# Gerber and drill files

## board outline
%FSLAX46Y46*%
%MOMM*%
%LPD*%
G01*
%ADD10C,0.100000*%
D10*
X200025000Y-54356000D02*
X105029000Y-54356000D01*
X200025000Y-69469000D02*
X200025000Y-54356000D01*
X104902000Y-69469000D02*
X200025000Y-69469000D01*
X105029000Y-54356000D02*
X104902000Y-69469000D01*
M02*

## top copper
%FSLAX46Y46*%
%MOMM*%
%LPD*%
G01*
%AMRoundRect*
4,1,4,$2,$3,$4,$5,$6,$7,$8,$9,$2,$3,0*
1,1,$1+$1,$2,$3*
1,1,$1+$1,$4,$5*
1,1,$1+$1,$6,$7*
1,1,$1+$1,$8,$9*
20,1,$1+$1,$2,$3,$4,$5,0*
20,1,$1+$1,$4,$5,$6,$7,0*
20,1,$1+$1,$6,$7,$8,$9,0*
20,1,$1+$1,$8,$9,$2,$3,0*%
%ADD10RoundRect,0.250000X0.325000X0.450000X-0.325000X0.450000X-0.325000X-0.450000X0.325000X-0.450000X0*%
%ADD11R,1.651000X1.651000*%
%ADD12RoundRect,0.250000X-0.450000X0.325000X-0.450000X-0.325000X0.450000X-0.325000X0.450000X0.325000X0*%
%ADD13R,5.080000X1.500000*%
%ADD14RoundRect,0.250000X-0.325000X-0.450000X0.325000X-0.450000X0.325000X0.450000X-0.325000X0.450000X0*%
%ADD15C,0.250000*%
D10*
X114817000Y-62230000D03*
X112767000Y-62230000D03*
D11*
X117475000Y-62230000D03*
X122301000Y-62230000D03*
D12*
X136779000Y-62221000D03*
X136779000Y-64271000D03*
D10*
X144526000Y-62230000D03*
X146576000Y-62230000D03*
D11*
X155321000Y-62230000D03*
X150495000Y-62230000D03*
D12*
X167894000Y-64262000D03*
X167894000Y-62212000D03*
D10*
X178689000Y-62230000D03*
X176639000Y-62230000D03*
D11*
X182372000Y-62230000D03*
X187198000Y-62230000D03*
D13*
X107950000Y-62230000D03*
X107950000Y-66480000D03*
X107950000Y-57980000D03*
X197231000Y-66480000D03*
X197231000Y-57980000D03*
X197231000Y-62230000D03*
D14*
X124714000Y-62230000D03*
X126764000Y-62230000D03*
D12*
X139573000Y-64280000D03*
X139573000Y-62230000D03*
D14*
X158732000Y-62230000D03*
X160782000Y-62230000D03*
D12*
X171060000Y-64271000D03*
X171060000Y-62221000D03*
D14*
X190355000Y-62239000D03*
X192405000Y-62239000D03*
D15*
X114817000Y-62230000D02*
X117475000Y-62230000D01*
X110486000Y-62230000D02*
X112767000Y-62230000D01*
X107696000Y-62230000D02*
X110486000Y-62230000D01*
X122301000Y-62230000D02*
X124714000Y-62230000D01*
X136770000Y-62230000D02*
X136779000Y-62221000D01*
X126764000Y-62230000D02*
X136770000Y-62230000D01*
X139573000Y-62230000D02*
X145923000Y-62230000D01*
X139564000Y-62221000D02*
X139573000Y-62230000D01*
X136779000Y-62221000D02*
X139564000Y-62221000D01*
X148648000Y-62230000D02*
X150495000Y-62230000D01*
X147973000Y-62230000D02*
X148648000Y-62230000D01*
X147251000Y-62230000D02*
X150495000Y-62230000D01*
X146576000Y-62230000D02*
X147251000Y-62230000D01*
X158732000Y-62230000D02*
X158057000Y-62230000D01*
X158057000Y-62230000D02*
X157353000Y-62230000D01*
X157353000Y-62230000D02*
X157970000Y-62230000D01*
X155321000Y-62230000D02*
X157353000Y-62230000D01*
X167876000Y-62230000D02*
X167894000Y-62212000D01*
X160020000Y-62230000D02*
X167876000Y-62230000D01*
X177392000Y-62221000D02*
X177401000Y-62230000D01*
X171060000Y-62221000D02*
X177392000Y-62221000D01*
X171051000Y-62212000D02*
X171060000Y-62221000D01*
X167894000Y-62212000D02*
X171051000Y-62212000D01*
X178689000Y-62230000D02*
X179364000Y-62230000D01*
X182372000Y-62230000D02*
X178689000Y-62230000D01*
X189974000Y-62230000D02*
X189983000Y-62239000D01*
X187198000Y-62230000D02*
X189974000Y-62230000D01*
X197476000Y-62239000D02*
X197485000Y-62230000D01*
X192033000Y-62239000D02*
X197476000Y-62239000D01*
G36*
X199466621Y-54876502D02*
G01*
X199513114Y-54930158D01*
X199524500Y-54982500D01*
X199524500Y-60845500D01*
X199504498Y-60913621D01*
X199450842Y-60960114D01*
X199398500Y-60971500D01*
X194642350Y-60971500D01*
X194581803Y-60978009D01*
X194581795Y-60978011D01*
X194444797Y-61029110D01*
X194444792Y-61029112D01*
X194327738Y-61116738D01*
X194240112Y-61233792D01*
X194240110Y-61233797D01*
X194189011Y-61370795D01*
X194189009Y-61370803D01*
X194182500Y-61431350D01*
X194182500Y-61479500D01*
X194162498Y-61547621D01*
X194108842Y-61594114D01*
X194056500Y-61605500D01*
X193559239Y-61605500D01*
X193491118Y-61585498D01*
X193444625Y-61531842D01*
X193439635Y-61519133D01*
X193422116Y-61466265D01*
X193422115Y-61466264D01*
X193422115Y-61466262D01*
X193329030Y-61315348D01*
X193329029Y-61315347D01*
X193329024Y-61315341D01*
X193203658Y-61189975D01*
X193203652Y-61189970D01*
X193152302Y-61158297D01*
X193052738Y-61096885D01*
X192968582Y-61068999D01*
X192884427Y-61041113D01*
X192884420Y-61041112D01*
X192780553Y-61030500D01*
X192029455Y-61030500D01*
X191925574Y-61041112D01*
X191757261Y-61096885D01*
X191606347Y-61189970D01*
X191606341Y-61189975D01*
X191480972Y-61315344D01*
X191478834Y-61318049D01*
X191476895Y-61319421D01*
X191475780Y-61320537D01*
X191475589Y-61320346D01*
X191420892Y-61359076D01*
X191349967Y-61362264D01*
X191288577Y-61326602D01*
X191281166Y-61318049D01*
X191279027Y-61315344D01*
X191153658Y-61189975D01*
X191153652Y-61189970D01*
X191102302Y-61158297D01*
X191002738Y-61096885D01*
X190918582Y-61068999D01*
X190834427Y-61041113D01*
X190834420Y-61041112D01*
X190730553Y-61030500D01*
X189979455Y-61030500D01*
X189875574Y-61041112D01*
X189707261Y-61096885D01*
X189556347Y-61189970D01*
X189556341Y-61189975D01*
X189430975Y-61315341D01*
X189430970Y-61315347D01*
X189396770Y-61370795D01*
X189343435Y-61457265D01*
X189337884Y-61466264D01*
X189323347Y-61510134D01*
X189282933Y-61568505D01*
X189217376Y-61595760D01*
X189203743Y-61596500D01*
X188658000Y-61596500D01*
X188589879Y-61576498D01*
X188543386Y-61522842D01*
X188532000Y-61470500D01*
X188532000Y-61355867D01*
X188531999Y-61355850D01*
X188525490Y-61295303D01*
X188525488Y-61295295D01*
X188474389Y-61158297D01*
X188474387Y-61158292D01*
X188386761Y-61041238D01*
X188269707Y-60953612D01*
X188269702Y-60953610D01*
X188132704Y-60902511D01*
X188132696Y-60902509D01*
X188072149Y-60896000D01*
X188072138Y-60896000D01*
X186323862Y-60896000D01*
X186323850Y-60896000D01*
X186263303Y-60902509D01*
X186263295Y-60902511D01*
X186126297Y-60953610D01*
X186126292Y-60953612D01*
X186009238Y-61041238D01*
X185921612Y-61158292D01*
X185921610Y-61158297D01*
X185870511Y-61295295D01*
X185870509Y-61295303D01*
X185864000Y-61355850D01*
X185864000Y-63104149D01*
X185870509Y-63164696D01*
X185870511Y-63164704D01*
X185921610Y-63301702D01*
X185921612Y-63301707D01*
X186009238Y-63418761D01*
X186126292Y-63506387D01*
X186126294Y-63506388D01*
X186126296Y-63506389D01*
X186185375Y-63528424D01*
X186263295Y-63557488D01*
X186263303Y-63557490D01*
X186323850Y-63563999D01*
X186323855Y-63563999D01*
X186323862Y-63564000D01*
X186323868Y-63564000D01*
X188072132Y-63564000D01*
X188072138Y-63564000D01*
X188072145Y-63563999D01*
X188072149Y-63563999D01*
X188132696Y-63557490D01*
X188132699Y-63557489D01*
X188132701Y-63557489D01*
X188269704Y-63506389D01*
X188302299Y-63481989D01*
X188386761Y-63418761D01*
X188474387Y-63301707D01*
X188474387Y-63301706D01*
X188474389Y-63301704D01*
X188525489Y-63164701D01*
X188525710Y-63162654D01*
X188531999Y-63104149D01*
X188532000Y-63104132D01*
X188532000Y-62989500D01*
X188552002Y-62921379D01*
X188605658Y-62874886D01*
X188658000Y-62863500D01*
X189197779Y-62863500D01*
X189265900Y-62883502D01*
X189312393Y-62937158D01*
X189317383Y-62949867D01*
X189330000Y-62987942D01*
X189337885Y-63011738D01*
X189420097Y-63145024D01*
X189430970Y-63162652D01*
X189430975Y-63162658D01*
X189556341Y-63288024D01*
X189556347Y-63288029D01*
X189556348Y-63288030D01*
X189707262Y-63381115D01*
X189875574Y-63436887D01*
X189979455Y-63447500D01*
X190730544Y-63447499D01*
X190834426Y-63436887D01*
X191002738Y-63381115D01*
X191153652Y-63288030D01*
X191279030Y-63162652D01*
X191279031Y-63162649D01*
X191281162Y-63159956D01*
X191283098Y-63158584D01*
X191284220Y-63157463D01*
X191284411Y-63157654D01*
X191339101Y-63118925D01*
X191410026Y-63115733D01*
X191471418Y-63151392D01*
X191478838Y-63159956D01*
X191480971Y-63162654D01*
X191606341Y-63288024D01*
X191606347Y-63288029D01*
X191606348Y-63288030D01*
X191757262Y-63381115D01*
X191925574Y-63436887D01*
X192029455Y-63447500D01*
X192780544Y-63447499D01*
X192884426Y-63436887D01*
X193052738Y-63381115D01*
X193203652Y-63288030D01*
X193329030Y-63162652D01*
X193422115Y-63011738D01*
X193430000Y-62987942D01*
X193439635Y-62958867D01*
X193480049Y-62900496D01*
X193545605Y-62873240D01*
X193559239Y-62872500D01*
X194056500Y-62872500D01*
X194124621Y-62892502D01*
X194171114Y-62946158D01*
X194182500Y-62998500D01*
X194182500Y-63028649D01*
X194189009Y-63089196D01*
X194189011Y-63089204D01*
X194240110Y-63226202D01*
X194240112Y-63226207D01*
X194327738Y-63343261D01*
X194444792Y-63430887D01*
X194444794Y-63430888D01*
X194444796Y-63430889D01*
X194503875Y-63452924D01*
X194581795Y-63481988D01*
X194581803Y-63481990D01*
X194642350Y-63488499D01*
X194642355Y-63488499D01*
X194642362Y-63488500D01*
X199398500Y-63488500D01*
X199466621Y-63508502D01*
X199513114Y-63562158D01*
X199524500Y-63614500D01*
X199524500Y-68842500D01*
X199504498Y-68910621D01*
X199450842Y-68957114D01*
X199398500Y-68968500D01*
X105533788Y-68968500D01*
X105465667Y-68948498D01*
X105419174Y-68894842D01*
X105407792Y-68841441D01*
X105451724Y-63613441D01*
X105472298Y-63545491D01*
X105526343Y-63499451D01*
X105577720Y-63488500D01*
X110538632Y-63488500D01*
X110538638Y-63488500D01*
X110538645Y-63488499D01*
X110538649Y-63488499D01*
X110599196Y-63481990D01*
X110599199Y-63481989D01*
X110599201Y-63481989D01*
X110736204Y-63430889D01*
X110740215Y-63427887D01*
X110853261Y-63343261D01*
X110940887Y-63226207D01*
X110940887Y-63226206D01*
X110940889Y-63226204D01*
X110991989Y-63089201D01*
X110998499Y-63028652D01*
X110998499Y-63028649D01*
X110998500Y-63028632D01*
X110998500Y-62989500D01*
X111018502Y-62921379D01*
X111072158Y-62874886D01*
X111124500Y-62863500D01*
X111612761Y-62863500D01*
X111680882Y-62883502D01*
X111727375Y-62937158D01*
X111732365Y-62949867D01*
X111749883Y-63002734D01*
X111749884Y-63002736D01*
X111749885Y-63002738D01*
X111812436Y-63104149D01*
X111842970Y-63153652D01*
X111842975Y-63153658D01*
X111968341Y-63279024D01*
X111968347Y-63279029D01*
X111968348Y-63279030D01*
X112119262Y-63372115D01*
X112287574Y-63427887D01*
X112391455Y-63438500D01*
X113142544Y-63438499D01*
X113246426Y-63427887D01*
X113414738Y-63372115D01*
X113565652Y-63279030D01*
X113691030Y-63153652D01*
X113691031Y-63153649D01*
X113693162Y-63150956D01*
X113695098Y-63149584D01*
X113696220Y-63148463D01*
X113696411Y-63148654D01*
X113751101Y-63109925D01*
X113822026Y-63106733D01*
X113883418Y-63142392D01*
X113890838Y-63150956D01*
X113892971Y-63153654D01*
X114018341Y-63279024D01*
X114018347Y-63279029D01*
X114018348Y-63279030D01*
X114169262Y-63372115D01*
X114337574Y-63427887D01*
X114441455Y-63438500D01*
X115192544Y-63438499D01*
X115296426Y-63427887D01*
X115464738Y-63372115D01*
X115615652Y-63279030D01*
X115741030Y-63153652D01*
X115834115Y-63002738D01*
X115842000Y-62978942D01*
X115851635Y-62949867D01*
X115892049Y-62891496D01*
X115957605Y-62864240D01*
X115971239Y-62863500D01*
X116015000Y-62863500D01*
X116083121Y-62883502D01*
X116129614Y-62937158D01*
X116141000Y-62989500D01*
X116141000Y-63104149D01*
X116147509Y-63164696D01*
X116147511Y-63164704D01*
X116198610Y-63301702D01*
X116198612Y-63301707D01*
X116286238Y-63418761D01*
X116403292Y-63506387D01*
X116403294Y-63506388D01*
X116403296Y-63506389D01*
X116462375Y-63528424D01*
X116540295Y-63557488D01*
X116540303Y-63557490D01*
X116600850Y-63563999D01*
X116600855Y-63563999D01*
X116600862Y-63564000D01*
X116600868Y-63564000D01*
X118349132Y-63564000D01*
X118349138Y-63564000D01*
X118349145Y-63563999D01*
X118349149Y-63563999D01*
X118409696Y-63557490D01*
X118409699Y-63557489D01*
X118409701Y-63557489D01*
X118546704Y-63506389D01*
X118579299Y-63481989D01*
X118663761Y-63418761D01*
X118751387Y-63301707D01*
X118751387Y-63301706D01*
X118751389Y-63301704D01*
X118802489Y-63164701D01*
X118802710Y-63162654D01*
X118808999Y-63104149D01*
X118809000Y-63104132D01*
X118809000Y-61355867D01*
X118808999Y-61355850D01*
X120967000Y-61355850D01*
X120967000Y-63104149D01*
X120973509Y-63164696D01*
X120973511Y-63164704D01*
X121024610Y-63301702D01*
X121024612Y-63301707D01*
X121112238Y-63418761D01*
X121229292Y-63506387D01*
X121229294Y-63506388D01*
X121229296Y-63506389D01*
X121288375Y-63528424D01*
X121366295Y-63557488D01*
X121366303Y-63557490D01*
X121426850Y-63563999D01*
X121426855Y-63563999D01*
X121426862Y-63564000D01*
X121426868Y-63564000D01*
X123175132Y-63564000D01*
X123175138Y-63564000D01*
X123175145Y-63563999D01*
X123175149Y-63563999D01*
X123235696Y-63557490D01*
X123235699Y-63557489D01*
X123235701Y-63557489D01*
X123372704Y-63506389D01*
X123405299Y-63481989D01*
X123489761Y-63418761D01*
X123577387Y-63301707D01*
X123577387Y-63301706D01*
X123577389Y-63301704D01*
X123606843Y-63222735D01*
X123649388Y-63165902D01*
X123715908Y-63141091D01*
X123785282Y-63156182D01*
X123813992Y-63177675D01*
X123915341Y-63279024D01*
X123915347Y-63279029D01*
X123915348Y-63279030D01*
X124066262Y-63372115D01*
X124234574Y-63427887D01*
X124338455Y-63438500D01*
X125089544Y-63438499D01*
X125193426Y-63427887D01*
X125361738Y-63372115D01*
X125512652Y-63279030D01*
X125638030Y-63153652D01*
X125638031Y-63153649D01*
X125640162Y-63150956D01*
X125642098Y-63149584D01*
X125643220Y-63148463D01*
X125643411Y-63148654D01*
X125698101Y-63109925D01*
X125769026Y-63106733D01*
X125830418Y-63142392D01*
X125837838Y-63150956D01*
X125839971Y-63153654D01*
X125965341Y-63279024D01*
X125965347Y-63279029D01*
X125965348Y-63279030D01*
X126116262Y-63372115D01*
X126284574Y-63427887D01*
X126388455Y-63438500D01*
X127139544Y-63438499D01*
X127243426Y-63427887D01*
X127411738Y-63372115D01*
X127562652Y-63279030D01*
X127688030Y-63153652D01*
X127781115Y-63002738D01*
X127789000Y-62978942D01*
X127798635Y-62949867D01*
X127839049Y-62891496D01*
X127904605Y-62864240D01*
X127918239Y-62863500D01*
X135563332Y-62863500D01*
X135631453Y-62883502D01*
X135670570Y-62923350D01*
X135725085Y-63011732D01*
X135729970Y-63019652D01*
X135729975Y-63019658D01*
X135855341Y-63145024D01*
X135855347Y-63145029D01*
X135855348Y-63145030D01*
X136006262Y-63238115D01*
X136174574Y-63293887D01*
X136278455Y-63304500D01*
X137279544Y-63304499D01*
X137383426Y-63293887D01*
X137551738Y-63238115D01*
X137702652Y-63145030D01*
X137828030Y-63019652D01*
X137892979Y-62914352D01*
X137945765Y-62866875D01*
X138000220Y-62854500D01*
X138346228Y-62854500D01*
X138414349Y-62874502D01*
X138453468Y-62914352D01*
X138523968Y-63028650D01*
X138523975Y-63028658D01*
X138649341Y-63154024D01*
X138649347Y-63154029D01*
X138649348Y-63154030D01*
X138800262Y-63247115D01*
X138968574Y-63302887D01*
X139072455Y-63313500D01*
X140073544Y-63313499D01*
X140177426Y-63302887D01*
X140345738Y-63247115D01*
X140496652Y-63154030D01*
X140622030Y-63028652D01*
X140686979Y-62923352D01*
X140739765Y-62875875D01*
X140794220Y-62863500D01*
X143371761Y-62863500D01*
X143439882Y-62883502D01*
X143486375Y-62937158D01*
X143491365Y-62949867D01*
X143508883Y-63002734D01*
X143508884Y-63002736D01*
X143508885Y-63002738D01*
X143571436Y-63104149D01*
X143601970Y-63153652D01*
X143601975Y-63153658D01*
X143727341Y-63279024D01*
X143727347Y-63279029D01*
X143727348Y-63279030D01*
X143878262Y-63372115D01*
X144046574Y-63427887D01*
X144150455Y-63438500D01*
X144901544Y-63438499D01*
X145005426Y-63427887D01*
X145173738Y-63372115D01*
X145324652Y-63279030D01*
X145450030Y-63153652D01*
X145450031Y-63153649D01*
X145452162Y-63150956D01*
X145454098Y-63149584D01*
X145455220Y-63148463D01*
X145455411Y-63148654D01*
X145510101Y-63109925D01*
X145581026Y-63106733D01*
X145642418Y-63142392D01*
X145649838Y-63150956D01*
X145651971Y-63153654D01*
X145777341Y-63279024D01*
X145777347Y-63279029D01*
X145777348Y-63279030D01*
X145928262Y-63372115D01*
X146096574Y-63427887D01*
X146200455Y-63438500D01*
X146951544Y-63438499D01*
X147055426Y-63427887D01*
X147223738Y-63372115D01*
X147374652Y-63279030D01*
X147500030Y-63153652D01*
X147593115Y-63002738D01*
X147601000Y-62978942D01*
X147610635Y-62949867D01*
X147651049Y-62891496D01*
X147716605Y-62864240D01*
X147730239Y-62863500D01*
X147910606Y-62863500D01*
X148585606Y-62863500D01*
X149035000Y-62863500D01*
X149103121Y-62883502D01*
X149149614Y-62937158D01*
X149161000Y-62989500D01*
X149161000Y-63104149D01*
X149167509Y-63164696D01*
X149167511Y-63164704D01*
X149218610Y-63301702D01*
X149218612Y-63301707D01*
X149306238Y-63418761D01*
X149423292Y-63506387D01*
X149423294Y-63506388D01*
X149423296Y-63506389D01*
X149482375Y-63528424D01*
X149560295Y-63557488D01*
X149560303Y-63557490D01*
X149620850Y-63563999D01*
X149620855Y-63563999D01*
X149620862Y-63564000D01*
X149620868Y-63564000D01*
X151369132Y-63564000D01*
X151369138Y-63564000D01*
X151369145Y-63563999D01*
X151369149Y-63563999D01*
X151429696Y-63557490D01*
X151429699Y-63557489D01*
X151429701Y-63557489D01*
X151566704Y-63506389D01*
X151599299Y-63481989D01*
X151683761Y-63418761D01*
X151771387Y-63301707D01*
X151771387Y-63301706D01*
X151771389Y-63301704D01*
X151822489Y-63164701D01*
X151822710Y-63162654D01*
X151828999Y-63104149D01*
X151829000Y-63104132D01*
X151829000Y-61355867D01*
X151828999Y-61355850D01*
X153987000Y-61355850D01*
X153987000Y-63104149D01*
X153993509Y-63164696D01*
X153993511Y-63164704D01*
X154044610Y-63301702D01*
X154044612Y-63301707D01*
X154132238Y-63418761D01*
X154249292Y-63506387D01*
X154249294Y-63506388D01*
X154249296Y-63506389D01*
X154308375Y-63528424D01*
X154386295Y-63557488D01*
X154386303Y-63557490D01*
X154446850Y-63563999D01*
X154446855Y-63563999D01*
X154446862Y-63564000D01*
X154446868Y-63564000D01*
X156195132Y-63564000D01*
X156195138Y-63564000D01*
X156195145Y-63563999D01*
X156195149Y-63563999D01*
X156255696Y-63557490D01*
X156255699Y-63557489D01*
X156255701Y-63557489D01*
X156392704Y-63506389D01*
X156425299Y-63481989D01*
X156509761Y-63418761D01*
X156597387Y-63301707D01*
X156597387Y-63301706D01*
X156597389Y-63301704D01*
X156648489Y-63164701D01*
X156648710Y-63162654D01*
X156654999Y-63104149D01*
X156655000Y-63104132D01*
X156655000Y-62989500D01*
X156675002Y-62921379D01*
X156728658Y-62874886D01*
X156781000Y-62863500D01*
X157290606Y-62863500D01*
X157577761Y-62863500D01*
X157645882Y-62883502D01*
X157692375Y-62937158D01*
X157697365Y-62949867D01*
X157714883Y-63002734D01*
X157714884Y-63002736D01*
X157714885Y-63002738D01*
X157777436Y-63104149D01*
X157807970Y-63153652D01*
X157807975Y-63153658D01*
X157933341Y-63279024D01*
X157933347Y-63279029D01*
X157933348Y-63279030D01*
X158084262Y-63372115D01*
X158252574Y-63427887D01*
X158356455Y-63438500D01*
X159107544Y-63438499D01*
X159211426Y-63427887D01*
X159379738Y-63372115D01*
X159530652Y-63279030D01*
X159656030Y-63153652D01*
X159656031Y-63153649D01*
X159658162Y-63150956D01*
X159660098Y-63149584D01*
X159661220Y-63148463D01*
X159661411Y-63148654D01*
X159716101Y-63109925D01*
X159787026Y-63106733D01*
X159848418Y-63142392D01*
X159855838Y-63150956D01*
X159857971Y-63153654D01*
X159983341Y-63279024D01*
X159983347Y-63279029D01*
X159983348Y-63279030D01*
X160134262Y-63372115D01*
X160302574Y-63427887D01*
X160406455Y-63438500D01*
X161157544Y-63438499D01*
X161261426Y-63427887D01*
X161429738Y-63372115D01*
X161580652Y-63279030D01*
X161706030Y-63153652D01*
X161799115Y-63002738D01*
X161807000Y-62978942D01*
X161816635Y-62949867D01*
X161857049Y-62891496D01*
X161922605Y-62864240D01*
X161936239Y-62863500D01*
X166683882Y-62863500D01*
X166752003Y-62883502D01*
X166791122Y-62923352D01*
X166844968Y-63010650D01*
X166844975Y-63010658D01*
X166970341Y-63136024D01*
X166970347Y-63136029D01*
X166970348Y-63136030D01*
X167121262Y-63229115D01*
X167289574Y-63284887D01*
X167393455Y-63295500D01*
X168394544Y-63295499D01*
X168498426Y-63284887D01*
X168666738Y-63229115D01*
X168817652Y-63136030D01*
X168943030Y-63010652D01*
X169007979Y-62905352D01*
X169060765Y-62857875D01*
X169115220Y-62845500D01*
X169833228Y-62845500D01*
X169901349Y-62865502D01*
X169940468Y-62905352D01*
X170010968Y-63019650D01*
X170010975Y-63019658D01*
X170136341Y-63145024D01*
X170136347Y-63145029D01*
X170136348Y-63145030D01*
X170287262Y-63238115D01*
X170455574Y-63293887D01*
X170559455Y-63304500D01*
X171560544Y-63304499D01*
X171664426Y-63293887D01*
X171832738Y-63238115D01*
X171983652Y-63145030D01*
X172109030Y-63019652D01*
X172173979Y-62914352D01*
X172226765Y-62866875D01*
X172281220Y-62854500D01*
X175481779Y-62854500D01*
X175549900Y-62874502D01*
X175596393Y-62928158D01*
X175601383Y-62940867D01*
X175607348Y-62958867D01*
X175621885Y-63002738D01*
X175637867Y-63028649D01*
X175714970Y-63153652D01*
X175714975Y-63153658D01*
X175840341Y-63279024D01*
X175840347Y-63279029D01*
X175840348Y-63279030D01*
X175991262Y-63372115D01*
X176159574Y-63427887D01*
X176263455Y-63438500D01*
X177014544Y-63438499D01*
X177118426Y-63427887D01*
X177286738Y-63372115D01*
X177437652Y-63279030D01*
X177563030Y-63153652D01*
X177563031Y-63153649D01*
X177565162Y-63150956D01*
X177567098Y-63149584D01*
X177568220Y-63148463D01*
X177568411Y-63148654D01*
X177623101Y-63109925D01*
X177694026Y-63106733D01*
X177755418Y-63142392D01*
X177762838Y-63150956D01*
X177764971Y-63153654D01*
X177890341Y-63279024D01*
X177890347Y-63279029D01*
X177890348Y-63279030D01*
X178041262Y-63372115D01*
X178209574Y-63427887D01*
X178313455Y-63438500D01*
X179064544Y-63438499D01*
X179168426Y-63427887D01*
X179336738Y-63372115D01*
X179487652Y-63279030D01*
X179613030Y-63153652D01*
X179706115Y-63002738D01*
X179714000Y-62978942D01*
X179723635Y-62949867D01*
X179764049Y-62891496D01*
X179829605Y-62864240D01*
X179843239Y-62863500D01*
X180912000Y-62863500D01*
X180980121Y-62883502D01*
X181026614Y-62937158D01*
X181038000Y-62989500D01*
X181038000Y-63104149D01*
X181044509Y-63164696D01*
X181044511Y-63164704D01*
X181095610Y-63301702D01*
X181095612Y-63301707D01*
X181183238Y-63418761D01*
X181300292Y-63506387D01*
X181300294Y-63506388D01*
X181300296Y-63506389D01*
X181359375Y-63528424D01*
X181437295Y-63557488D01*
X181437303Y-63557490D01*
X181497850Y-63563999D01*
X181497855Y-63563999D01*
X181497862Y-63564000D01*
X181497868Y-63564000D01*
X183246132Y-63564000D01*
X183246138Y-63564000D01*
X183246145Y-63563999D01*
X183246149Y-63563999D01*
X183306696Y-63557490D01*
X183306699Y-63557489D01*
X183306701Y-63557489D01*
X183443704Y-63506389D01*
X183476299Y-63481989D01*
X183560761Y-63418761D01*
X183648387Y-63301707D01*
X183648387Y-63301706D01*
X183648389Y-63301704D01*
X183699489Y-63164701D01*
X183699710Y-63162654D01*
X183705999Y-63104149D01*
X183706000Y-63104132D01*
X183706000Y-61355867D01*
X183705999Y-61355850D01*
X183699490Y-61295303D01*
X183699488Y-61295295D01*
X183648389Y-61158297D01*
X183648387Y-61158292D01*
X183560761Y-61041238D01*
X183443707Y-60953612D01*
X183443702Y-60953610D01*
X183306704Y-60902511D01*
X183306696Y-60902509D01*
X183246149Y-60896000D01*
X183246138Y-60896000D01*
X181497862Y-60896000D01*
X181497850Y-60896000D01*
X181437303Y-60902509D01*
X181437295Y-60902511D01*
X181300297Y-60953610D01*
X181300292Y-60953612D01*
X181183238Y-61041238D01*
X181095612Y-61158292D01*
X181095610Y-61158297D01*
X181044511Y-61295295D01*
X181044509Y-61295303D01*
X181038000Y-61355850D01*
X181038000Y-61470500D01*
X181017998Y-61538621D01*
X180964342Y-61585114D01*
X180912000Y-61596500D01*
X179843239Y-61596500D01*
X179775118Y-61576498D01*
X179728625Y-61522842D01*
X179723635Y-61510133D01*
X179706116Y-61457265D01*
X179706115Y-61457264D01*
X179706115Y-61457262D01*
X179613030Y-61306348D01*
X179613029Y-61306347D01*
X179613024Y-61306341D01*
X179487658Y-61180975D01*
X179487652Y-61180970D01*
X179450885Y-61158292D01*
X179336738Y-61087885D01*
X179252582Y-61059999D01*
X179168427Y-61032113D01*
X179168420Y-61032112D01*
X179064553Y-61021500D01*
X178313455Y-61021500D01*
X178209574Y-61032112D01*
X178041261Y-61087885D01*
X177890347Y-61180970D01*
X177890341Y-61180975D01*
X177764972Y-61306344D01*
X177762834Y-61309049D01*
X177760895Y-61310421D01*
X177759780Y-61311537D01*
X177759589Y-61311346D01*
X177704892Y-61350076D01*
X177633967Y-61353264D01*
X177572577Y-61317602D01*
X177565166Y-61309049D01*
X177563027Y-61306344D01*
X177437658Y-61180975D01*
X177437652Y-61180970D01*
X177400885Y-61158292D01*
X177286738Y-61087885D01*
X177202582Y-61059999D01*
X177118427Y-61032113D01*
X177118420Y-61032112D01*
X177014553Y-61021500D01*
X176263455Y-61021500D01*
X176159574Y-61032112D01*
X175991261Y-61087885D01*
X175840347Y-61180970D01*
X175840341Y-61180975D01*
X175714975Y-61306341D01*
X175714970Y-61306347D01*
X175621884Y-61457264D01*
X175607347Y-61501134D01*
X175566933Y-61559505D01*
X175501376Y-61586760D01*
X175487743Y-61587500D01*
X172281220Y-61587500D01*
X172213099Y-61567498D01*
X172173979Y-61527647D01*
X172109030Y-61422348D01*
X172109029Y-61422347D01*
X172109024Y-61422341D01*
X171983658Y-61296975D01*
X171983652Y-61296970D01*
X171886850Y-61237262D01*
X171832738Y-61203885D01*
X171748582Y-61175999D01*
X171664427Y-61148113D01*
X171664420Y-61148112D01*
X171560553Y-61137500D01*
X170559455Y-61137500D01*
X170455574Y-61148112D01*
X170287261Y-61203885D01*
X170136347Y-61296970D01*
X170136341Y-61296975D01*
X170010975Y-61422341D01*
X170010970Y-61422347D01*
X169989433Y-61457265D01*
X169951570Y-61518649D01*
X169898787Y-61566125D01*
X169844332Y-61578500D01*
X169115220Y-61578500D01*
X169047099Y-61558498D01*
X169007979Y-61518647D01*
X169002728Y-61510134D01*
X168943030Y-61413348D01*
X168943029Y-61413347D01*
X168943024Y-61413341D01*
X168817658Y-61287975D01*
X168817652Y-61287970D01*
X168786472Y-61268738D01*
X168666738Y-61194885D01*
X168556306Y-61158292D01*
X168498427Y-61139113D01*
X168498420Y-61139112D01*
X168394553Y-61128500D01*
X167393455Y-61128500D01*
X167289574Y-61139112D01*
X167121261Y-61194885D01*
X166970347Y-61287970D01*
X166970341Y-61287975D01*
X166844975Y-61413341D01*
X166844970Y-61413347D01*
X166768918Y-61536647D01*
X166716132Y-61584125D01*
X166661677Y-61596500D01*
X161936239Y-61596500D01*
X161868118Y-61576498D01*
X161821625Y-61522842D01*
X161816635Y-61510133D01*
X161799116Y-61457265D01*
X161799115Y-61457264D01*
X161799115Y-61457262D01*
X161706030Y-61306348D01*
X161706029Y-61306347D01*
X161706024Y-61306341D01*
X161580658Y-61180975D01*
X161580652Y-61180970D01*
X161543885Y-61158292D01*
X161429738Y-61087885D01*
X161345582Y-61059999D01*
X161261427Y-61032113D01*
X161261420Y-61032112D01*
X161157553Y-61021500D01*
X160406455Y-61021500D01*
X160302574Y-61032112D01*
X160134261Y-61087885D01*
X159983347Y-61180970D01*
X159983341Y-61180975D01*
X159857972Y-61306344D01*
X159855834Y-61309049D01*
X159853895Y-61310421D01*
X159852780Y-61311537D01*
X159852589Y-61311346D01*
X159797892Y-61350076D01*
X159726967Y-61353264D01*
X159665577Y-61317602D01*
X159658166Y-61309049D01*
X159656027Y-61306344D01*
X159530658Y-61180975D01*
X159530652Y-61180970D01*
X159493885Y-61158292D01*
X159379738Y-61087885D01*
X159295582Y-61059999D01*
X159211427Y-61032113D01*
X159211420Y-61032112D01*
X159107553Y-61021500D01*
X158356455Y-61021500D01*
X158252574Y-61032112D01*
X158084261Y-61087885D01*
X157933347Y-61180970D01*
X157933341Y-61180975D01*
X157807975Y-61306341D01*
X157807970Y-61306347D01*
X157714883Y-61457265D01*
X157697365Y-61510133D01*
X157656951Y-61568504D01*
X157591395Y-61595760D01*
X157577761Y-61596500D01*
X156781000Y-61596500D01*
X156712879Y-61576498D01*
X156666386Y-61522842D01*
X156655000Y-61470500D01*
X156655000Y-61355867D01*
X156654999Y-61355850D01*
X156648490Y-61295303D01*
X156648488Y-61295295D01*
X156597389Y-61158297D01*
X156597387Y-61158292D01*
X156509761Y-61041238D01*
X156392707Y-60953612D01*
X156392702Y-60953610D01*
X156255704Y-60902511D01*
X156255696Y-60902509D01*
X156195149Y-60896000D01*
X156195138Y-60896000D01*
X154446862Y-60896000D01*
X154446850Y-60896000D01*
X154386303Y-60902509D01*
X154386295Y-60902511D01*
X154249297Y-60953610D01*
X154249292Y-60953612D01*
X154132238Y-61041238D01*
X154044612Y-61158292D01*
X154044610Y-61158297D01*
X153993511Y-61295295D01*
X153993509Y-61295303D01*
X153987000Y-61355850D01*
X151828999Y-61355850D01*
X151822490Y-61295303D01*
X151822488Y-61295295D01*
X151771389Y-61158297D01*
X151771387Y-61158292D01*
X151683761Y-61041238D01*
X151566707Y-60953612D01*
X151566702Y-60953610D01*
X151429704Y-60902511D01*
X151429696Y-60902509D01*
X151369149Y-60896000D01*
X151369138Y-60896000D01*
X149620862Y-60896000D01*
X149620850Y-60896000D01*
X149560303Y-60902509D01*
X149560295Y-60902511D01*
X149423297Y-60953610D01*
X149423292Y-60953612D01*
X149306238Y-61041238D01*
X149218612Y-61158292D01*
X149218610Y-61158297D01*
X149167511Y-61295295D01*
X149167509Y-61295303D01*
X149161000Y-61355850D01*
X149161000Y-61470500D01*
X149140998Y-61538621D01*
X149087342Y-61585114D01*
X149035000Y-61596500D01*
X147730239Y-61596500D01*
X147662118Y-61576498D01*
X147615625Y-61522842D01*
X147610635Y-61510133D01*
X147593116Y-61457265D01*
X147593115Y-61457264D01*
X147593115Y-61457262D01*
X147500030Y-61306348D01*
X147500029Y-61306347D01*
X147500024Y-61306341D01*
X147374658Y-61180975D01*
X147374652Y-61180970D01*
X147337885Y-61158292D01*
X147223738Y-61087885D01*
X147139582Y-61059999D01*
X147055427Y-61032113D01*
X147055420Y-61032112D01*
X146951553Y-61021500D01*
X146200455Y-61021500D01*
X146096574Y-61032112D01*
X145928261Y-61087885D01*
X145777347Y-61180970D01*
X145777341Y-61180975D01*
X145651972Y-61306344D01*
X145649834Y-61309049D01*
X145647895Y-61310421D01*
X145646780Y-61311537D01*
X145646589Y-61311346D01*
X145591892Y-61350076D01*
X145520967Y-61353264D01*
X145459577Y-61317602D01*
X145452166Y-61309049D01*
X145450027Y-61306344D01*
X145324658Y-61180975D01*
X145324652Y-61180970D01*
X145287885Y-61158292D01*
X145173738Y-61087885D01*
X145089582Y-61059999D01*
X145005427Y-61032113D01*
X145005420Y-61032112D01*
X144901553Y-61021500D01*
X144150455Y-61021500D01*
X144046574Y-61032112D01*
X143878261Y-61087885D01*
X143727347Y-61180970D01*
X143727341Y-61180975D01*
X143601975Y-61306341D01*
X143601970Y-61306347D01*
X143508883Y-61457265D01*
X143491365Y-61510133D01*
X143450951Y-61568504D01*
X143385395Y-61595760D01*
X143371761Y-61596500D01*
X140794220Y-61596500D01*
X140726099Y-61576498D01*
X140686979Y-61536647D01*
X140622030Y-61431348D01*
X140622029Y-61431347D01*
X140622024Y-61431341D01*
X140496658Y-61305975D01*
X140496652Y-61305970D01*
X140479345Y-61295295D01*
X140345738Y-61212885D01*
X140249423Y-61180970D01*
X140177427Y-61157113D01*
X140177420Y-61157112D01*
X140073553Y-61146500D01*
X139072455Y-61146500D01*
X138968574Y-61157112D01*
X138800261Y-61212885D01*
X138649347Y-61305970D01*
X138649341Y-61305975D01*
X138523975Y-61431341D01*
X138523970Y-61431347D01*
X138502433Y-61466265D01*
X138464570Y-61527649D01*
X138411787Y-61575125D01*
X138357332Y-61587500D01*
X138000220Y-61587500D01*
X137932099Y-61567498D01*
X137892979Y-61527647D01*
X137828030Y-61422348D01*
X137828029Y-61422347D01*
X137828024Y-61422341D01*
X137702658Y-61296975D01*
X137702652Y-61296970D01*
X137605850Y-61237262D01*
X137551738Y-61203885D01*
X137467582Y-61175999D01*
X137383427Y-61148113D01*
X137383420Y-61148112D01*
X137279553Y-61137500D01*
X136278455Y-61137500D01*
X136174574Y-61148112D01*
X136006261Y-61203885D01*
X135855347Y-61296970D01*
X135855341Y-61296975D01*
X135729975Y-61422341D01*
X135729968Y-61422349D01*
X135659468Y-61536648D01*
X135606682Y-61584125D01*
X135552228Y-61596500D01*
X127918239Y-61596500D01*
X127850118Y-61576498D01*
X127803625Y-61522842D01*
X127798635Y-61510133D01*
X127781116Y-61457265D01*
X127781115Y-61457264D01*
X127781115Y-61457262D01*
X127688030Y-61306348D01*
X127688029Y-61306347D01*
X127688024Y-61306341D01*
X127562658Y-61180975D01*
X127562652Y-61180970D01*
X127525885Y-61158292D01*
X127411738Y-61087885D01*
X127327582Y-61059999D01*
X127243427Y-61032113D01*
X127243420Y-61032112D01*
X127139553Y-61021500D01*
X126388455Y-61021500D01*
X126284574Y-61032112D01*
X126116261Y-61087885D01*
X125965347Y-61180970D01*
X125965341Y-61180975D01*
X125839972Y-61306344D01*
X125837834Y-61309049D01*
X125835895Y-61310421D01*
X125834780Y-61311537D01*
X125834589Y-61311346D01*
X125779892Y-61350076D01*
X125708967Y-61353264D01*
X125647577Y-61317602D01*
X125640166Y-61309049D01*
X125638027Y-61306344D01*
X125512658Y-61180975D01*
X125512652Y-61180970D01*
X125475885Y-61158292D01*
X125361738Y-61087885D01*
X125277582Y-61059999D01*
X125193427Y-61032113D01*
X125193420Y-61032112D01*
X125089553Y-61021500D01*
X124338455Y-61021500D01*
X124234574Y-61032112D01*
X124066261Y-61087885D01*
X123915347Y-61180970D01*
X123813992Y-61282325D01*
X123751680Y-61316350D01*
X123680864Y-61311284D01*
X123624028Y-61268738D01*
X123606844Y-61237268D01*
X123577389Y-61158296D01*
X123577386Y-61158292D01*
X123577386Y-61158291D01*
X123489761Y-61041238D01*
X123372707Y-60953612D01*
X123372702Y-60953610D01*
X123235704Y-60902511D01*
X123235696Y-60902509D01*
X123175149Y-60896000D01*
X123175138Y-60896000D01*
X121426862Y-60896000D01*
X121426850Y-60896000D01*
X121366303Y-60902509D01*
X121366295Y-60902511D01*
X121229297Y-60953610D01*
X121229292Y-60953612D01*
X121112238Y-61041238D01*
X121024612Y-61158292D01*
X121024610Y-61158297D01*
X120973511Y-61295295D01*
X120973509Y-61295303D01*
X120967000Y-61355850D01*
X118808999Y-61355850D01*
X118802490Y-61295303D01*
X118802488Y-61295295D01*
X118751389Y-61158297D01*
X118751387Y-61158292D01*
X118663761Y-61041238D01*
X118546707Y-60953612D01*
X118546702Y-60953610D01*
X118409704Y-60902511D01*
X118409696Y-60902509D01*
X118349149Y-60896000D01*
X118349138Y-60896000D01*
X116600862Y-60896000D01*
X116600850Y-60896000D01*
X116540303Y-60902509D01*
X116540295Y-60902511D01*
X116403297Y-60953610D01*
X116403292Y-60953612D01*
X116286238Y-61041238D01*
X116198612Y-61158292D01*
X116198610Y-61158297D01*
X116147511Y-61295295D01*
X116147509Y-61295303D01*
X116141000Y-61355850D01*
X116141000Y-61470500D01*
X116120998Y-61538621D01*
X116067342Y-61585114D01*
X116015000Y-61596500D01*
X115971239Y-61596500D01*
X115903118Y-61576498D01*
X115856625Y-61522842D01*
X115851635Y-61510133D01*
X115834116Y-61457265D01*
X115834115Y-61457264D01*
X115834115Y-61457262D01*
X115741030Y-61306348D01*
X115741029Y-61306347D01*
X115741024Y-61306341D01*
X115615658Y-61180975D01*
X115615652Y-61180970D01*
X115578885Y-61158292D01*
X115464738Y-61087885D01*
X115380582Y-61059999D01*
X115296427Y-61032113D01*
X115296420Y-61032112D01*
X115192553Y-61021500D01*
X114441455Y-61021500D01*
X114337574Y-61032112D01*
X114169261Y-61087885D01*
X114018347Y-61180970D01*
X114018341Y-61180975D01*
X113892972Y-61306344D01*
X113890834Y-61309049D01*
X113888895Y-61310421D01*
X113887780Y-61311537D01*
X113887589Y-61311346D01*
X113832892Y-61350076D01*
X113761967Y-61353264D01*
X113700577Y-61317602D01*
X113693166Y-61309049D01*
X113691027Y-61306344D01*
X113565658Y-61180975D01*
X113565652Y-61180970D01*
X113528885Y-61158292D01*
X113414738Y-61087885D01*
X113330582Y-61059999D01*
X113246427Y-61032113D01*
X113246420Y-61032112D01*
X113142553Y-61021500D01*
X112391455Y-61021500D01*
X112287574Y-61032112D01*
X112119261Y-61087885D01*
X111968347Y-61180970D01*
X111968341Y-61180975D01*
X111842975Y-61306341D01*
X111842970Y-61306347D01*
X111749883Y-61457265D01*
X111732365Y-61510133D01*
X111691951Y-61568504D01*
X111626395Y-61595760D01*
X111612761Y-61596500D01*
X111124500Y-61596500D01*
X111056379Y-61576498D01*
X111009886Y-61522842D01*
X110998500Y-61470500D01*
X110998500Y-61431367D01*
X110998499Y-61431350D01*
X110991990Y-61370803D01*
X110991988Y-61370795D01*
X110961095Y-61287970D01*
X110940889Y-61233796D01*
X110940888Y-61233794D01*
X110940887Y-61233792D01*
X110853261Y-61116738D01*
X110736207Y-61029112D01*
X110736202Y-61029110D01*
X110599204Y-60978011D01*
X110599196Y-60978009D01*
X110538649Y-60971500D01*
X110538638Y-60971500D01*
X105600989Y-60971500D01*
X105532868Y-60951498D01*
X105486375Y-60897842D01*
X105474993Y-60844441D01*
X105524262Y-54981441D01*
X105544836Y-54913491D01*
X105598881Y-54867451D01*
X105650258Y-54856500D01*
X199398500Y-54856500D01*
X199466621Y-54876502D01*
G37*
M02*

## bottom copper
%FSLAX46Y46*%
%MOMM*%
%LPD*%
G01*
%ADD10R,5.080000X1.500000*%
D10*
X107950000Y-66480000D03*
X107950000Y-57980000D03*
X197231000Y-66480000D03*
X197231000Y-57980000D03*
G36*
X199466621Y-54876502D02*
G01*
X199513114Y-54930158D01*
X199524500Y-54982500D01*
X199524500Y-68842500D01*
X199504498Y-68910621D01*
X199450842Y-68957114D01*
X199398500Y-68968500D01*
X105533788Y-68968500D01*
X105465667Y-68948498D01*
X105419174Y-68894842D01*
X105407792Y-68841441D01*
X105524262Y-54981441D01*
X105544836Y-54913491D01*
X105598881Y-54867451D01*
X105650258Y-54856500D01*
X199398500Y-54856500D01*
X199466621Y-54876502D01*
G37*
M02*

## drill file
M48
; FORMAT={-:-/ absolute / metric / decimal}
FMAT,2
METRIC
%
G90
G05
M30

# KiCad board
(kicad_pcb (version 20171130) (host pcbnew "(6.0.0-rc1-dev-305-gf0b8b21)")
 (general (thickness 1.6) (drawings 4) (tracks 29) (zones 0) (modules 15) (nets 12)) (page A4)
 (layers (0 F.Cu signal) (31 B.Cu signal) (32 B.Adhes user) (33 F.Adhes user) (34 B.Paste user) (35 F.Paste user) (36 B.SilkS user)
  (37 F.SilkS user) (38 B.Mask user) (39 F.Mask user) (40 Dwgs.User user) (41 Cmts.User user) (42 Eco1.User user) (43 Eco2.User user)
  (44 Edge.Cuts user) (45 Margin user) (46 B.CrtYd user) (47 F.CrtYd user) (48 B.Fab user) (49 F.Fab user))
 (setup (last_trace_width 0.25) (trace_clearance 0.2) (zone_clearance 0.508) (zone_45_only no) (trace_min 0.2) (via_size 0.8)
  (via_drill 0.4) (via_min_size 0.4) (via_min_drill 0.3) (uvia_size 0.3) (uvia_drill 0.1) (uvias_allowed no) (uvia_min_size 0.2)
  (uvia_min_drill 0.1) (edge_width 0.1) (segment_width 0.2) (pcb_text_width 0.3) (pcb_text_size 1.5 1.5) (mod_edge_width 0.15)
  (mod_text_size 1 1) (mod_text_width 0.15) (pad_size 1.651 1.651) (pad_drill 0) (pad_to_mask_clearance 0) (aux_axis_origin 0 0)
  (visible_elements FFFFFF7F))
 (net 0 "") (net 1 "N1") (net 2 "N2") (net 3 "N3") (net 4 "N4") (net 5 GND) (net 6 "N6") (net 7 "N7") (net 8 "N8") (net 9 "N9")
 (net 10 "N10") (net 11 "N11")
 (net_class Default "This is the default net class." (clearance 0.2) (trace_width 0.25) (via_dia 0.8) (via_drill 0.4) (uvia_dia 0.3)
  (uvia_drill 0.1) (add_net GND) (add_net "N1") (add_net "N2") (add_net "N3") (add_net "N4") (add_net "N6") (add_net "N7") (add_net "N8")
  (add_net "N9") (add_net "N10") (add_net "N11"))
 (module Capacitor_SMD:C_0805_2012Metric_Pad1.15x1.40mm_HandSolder (layer F.Cu) (at 113.792 62.23 180)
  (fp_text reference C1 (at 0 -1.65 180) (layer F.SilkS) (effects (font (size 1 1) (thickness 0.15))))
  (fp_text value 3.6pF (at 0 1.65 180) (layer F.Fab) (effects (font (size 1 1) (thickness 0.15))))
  (pad 1 smd roundrect (at -1.025 0 180) (size 1.15 1.4) (layers F.Cu F.Paste F.Mask) (roundrect_rratio 0.217391) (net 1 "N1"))
  (pad 2 smd roundrect (at 1.025 0 180) (size 1.15 1.4) (layers F.Cu F.Paste F.Mask) (roundrect_rratio 0.217391) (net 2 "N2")))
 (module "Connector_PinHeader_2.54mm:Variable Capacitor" (layer F.Cu) (at 119.507 62.23)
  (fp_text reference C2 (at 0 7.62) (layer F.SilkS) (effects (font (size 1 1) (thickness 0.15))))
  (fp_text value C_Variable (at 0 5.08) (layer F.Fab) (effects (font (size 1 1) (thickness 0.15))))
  (pad 1 smd rect (at -2.032 0) (size 1.651 1.651) (layers F.Cu F.Paste F.Mask) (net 1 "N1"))
  (pad 2 smd rect (at 2.794 0) (size 1.651 1.651) (layers F.Cu F.Paste F.Mask) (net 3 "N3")))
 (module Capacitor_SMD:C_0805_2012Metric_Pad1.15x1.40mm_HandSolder (layer F.Cu) (at 136.779 63.246 270)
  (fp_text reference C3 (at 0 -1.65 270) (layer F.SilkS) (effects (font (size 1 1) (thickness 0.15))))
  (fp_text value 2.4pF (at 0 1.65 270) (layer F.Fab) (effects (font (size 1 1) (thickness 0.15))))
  (pad 1 smd roundrect (at -1.025 0 270) (size 1.15 1.4) (layers F.Cu F.Paste F.Mask) (roundrect_rratio 0.217391) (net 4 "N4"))
  (pad 2 smd roundrect (at 1.025 0 270) (size 1.15 1.4) (layers F.Cu F.Paste F.Mask) (roundrect_rratio 0.217391) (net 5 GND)))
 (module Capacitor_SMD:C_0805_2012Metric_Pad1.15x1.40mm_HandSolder (layer F.Cu) (at 145.551 62.23 180)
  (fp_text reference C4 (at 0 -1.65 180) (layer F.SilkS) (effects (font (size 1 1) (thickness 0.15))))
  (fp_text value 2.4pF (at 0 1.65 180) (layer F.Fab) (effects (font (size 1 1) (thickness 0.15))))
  (pad 2 smd roundrect (at 1.025 0 180) (size 1.15 1.4) (layers F.Cu F.Paste F.Mask) (roundrect_rratio 0.217391) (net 4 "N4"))
  (pad 1 smd roundrect (at -1.025 0 180) (size 1.15 1.4) (layers F.Cu F.Paste F.Mask) (roundrect_rratio 0.217391) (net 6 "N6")))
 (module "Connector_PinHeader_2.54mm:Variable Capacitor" (layer F.Cu) (at 152.527 62.23)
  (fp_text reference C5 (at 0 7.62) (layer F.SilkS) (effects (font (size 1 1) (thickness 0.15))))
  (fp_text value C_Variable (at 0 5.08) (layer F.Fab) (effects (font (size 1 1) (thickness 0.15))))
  (pad 2 smd rect (at 2.794 0) (size 1.651 1.651) (layers F.Cu F.Paste F.Mask) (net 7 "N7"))
  (pad 1 smd rect (at -2.032 0) (size 1.651 1.651) (layers F.Cu F.Paste F.Mask) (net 6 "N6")))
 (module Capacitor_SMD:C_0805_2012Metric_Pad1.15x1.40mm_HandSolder (layer F.Cu) (at 167.894 63.237 270)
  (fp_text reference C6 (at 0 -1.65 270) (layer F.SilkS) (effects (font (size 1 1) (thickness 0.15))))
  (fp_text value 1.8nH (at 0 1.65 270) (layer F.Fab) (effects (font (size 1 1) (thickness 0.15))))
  (pad 2 smd roundrect (at 1.025 0 270) (size 1.15 1.4) (layers F.Cu F.Paste F.Mask) (roundrect_rratio 0.217391) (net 5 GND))
  (pad 1 smd roundrect (at -1.025 0 270) (size 1.15 1.4) (layers F.Cu F.Paste F.Mask) (roundrect_rratio 0.217391) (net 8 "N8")))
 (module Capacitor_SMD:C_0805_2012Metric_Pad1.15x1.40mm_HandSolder (layer F.Cu) (at 177.664 62.23 180)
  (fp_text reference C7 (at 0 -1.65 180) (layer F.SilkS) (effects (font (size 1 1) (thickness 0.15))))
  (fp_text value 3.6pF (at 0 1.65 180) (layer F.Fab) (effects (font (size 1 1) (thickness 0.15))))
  (pad 1 smd roundrect (at -1.025 0 180) (size 1.15 1.4) (layers F.Cu F.Paste F.Mask) (roundrect_rratio 0.217391) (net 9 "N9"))
  (pad 2 smd roundrect (at 1.025 0 180) (size 1.15 1.4) (layers F.Cu F.Paste F.Mask) (roundrect_rratio 0.217391) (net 8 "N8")))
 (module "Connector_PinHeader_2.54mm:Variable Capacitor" (layer F.Cu) (at 184.404 62.23)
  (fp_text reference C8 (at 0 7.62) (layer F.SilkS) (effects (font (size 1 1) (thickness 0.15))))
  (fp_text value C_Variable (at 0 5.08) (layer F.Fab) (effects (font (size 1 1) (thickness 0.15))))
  (pad 1 smd rect (at -2.032 0) (size 1.651 1.651) (layers F.Cu F.Paste F.Mask) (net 9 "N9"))
  (pad 2 smd rect (at 2.794 0) (size 1.651 1.651) (layers F.Cu F.Paste F.Mask) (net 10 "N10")))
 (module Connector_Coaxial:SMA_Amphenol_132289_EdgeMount (layer F.Cu) (at 107.95 62.23 180)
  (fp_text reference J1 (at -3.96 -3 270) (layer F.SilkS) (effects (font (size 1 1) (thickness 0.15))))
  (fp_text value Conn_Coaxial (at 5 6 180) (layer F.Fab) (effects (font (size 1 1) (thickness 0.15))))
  (pad 1 smd rect (at 0 0 270) (size 1.5 5.08) (layers F.Cu F.Paste F.Mask) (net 2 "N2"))
  (pad 2 smd rect (at 0 -4.25 270) (size 1.5 5.08) (layers F.Cu F.Paste F.Mask) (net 5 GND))
  (pad 2 smd rect (at 0 4.25 270) (size 1.5 5.08) (layers F.Cu F.Paste F.Mask) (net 5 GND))
  (pad 2 smd rect (at 0 -4.25 270) (size 1.5 5.08) (layers B.Cu B.Paste B.Mask) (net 5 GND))
  (pad 2 smd rect (at 0 4.25 270) (size 1.5 5.08) (layers B.Cu B.Paste B.Mask) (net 5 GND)))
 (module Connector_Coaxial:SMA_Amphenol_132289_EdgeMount (layer F.Cu) (at 197.231 62.23)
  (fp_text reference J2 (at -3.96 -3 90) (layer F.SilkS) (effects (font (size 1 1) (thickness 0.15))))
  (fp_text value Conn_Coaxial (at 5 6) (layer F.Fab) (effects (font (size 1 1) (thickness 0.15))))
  (pad 2 smd rect (at 0 4.25 90) (size 1.5 5.08) (layers B.Cu B.Paste B.Mask) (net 5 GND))
  (pad 2 smd rect (at 0 -4.25 90) (size 1.5 5.08) (layers B.Cu B.Paste B.Mask) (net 5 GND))
  (pad 2 smd rect (at 0 4.25 90) (size 1.5 5.08) (layers F.Cu F.Paste F.Mask) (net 5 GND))
  (pad 2 smd rect (at 0 -4.25 90) (size 1.5 5.08) (layers F.Cu F.Paste F.Mask) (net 5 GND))
  (pad 1 smd rect (at 0 0 90) (size 1.5 5.08) (layers F.Cu F.Paste F.Mask) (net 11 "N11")))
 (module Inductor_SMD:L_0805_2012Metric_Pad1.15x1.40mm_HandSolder (layer F.Cu) (at 125.739 62.23)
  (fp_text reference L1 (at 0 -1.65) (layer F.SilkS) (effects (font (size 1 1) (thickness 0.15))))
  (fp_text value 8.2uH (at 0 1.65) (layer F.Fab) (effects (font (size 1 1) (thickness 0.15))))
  (pad 1 smd roundrect (at -1.025 0) (size 1.15 1.4) (layers F.Cu F.Paste F.Mask) (roundrect_rratio 0.217391) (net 3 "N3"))
  (pad 2 smd roundrect (at 1.025 0) (size 1.15 1.4) (layers F.Cu F.Paste F.Mask) (roundrect_rratio 0.217391) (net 4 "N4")))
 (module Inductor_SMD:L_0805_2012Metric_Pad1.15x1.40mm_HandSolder (layer F.Cu) (at 139.573 63.255 270)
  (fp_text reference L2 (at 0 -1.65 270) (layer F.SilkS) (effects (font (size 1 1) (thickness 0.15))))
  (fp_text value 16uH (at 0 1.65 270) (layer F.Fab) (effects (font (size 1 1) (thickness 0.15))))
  (pad 2 smd roundrect (at 1.025 0 270) (size 1.15 1.4) (layers F.Cu F.Paste F.Mask) (roundrect_rratio 0.217391) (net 5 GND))
  (pad 1 smd roundrect (at -1.025 0 270) (size 1.15 1.4) (layers F.Cu F.Paste F.Mask) (roundrect_rratio 0.217391) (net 4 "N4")))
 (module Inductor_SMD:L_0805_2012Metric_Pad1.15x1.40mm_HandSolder (layer F.Cu) (at 159.757 62.23)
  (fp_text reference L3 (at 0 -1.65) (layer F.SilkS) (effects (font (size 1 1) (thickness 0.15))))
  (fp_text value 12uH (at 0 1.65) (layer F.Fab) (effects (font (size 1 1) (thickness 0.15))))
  (pad 1 smd roundrect (at -1.025 0) (size 1.15 1.4) (layers F.Cu F.Paste F.Mask) (roundrect_rratio 0.217391) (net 7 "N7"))
  (pad 2 smd roundrect (at 1.025 0) (size 1.15 1.4) (layers F.Cu F.Paste F.Mask) (roundrect_rratio 0.217391) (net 8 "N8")))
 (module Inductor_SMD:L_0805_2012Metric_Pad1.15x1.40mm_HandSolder (layer F.Cu) (at 171.06 63.246 270)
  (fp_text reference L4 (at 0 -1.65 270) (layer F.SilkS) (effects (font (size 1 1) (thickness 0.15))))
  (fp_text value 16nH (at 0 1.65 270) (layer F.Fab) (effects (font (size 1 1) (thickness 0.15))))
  (pad 2 smd roundrect (at 1.025 0 270) (size 1.15 1.4) (layers F.Cu F.Paste F.Mask) (roundrect_rratio 0.217391) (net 5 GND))
  (pad 1 smd roundrect (at -1.025 0 270) (size 1.15 1.4) (layers F.Cu F.Paste F.Mask) (roundrect_rratio 0.217391) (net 8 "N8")))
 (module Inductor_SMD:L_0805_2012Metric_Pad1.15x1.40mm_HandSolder (layer F.Cu) (at 191.38 62.239)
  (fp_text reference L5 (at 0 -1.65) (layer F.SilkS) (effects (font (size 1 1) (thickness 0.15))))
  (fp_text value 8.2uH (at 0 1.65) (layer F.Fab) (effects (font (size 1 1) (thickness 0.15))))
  (pad 1 smd roundrect (at -1.025 0) (size 1.15 1.4) (layers F.Cu F.Paste F.Mask) (roundrect_rratio 0.217391) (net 10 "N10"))
  (pad 2 smd roundrect (at 1.025 0) (size 1.15 1.4) (layers F.Cu F.Paste F.Mask) (roundrect_rratio 0.217391) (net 11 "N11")))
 (gr_line (start 200.025 54.356) (end 105.029 54.356) (layer Edge.Cuts) (width 0.1))
 (gr_line (start 200.025 69.469) (end 200.025 54.356) (layer Edge.Cuts) (width 0.1))
 (gr_line (start 104.902 69.469) (end 200.025 69.469) (layer Edge.Cuts) (width 0.1))
 (gr_line (start 105.029 54.356) (end 104.902 69.469) (layer Edge.Cuts) (width 0.1))
 (segment (start 114.817 62.23) (end 117.475 62.23) (width 0.25) (layer F.Cu) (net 1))
 (segment (start 110.486 62.23) (end 112.767 62.23) (width 0.25) (layer F.Cu) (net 2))
 (segment (start 107.696 62.23) (end 110.486 62.23) (width 0.25) (layer F.Cu) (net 2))
 (segment (start 122.301 62.23) (end 124.714 62.23) (width 0.25) (layer F.Cu) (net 3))
 (segment (start 136.77 62.23) (end 136.779 62.221) (width 0.25) (layer F.Cu) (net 4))
 (segment (start 126.764 62.23) (end 136.77 62.23) (width 0.25) (layer F.Cu) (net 4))
 (segment (start 139.573 62.23) (end 145.923 62.23) (width 0.25) (layer F.Cu) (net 4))
 (segment (start 139.564 62.221) (end 139.573 62.23) (width 0.25) (layer F.Cu) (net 4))
 (segment (start 136.779 62.221) (end 139.564 62.221) (width 0.25) (layer F.Cu) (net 4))
 (segment (start 148.648 62.23) (end 150.495 62.23) (width 0.25) (layer F.Cu) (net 6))
 (segment (start 147.973 62.23) (end 148.648 62.23) (width 0.25) (layer F.Cu) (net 6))
 (segment (start 147.251 62.23) (end 150.495 62.23) (width 0.25) (layer F.Cu) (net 6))
 (segment (start 146.576 62.23) (end 147.251 62.23) (width 0.25) (layer F.Cu) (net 6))
 (segment (start 158.732 62.23) (end 158.057 62.23) (width 0.25) (layer F.Cu) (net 7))
 (segment (start 158.057 62.23) (end 157.353 62.23) (width 0.25) (layer F.Cu) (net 7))
 (segment (start 157.353 62.23) (end 157.97 62.23) (width 0.25) (layer F.Cu) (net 7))
 (segment (start 155.321 62.23) (end 157.353 62.23) (width 0.25) (layer F.Cu) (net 7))
 (segment (start 167.876 62.23) (end 167.894 62.212) (width 0.25) (layer F.Cu) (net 8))
 (segment (start 160.02 62.23) (end 167.876 62.23) (width 0.25) (layer F.Cu) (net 8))
 (segment (start 177.392 62.221) (end 177.401 62.23) (width 0.25) (layer F.Cu) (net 8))
 (segment (start 171.06 62.221) (end 177.392 62.221) (width 0.25) (layer F.Cu) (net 8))
 (segment (start 171.051 62.212) (end 171.06 62.221) (width 0.25) (layer F.Cu) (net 8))
 (segment (start 167.894 62.212) (end 171.051 62.212) (width 0.25) (layer F.Cu) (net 8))
 (segment (start 178.689 62.23) (end 179.364 62.23) (width 0.25) (layer F.Cu) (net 9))
 (segment (start 182.372 62.23) (end 178.689 62.23) (width 0.25) (layer F.Cu) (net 9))
 (segment (start 189.974 62.23) (end 189.983 62.239) (width 0.25) (layer F.Cu) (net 10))
 (segment (start 187.198 62.23) (end 189.974 62.23) (width 0.25) (layer F.Cu) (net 10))
 (segment (start 197.476 62.239) (end 197.485 62.23) (width 0.25) (layer F.Cu) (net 11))
 (segment (start 192.033 62.239) (end 197.476 62.239) (width 0.25) (layer F.Cu) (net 11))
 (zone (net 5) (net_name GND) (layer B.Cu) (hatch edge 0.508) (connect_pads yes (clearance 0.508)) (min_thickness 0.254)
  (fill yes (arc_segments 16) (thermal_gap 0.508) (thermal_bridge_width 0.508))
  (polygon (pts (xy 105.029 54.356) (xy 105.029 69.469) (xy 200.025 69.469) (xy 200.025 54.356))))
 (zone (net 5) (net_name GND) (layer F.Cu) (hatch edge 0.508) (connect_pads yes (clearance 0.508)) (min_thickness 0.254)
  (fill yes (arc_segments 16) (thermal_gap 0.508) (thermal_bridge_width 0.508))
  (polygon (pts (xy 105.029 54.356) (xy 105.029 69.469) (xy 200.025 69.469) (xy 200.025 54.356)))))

